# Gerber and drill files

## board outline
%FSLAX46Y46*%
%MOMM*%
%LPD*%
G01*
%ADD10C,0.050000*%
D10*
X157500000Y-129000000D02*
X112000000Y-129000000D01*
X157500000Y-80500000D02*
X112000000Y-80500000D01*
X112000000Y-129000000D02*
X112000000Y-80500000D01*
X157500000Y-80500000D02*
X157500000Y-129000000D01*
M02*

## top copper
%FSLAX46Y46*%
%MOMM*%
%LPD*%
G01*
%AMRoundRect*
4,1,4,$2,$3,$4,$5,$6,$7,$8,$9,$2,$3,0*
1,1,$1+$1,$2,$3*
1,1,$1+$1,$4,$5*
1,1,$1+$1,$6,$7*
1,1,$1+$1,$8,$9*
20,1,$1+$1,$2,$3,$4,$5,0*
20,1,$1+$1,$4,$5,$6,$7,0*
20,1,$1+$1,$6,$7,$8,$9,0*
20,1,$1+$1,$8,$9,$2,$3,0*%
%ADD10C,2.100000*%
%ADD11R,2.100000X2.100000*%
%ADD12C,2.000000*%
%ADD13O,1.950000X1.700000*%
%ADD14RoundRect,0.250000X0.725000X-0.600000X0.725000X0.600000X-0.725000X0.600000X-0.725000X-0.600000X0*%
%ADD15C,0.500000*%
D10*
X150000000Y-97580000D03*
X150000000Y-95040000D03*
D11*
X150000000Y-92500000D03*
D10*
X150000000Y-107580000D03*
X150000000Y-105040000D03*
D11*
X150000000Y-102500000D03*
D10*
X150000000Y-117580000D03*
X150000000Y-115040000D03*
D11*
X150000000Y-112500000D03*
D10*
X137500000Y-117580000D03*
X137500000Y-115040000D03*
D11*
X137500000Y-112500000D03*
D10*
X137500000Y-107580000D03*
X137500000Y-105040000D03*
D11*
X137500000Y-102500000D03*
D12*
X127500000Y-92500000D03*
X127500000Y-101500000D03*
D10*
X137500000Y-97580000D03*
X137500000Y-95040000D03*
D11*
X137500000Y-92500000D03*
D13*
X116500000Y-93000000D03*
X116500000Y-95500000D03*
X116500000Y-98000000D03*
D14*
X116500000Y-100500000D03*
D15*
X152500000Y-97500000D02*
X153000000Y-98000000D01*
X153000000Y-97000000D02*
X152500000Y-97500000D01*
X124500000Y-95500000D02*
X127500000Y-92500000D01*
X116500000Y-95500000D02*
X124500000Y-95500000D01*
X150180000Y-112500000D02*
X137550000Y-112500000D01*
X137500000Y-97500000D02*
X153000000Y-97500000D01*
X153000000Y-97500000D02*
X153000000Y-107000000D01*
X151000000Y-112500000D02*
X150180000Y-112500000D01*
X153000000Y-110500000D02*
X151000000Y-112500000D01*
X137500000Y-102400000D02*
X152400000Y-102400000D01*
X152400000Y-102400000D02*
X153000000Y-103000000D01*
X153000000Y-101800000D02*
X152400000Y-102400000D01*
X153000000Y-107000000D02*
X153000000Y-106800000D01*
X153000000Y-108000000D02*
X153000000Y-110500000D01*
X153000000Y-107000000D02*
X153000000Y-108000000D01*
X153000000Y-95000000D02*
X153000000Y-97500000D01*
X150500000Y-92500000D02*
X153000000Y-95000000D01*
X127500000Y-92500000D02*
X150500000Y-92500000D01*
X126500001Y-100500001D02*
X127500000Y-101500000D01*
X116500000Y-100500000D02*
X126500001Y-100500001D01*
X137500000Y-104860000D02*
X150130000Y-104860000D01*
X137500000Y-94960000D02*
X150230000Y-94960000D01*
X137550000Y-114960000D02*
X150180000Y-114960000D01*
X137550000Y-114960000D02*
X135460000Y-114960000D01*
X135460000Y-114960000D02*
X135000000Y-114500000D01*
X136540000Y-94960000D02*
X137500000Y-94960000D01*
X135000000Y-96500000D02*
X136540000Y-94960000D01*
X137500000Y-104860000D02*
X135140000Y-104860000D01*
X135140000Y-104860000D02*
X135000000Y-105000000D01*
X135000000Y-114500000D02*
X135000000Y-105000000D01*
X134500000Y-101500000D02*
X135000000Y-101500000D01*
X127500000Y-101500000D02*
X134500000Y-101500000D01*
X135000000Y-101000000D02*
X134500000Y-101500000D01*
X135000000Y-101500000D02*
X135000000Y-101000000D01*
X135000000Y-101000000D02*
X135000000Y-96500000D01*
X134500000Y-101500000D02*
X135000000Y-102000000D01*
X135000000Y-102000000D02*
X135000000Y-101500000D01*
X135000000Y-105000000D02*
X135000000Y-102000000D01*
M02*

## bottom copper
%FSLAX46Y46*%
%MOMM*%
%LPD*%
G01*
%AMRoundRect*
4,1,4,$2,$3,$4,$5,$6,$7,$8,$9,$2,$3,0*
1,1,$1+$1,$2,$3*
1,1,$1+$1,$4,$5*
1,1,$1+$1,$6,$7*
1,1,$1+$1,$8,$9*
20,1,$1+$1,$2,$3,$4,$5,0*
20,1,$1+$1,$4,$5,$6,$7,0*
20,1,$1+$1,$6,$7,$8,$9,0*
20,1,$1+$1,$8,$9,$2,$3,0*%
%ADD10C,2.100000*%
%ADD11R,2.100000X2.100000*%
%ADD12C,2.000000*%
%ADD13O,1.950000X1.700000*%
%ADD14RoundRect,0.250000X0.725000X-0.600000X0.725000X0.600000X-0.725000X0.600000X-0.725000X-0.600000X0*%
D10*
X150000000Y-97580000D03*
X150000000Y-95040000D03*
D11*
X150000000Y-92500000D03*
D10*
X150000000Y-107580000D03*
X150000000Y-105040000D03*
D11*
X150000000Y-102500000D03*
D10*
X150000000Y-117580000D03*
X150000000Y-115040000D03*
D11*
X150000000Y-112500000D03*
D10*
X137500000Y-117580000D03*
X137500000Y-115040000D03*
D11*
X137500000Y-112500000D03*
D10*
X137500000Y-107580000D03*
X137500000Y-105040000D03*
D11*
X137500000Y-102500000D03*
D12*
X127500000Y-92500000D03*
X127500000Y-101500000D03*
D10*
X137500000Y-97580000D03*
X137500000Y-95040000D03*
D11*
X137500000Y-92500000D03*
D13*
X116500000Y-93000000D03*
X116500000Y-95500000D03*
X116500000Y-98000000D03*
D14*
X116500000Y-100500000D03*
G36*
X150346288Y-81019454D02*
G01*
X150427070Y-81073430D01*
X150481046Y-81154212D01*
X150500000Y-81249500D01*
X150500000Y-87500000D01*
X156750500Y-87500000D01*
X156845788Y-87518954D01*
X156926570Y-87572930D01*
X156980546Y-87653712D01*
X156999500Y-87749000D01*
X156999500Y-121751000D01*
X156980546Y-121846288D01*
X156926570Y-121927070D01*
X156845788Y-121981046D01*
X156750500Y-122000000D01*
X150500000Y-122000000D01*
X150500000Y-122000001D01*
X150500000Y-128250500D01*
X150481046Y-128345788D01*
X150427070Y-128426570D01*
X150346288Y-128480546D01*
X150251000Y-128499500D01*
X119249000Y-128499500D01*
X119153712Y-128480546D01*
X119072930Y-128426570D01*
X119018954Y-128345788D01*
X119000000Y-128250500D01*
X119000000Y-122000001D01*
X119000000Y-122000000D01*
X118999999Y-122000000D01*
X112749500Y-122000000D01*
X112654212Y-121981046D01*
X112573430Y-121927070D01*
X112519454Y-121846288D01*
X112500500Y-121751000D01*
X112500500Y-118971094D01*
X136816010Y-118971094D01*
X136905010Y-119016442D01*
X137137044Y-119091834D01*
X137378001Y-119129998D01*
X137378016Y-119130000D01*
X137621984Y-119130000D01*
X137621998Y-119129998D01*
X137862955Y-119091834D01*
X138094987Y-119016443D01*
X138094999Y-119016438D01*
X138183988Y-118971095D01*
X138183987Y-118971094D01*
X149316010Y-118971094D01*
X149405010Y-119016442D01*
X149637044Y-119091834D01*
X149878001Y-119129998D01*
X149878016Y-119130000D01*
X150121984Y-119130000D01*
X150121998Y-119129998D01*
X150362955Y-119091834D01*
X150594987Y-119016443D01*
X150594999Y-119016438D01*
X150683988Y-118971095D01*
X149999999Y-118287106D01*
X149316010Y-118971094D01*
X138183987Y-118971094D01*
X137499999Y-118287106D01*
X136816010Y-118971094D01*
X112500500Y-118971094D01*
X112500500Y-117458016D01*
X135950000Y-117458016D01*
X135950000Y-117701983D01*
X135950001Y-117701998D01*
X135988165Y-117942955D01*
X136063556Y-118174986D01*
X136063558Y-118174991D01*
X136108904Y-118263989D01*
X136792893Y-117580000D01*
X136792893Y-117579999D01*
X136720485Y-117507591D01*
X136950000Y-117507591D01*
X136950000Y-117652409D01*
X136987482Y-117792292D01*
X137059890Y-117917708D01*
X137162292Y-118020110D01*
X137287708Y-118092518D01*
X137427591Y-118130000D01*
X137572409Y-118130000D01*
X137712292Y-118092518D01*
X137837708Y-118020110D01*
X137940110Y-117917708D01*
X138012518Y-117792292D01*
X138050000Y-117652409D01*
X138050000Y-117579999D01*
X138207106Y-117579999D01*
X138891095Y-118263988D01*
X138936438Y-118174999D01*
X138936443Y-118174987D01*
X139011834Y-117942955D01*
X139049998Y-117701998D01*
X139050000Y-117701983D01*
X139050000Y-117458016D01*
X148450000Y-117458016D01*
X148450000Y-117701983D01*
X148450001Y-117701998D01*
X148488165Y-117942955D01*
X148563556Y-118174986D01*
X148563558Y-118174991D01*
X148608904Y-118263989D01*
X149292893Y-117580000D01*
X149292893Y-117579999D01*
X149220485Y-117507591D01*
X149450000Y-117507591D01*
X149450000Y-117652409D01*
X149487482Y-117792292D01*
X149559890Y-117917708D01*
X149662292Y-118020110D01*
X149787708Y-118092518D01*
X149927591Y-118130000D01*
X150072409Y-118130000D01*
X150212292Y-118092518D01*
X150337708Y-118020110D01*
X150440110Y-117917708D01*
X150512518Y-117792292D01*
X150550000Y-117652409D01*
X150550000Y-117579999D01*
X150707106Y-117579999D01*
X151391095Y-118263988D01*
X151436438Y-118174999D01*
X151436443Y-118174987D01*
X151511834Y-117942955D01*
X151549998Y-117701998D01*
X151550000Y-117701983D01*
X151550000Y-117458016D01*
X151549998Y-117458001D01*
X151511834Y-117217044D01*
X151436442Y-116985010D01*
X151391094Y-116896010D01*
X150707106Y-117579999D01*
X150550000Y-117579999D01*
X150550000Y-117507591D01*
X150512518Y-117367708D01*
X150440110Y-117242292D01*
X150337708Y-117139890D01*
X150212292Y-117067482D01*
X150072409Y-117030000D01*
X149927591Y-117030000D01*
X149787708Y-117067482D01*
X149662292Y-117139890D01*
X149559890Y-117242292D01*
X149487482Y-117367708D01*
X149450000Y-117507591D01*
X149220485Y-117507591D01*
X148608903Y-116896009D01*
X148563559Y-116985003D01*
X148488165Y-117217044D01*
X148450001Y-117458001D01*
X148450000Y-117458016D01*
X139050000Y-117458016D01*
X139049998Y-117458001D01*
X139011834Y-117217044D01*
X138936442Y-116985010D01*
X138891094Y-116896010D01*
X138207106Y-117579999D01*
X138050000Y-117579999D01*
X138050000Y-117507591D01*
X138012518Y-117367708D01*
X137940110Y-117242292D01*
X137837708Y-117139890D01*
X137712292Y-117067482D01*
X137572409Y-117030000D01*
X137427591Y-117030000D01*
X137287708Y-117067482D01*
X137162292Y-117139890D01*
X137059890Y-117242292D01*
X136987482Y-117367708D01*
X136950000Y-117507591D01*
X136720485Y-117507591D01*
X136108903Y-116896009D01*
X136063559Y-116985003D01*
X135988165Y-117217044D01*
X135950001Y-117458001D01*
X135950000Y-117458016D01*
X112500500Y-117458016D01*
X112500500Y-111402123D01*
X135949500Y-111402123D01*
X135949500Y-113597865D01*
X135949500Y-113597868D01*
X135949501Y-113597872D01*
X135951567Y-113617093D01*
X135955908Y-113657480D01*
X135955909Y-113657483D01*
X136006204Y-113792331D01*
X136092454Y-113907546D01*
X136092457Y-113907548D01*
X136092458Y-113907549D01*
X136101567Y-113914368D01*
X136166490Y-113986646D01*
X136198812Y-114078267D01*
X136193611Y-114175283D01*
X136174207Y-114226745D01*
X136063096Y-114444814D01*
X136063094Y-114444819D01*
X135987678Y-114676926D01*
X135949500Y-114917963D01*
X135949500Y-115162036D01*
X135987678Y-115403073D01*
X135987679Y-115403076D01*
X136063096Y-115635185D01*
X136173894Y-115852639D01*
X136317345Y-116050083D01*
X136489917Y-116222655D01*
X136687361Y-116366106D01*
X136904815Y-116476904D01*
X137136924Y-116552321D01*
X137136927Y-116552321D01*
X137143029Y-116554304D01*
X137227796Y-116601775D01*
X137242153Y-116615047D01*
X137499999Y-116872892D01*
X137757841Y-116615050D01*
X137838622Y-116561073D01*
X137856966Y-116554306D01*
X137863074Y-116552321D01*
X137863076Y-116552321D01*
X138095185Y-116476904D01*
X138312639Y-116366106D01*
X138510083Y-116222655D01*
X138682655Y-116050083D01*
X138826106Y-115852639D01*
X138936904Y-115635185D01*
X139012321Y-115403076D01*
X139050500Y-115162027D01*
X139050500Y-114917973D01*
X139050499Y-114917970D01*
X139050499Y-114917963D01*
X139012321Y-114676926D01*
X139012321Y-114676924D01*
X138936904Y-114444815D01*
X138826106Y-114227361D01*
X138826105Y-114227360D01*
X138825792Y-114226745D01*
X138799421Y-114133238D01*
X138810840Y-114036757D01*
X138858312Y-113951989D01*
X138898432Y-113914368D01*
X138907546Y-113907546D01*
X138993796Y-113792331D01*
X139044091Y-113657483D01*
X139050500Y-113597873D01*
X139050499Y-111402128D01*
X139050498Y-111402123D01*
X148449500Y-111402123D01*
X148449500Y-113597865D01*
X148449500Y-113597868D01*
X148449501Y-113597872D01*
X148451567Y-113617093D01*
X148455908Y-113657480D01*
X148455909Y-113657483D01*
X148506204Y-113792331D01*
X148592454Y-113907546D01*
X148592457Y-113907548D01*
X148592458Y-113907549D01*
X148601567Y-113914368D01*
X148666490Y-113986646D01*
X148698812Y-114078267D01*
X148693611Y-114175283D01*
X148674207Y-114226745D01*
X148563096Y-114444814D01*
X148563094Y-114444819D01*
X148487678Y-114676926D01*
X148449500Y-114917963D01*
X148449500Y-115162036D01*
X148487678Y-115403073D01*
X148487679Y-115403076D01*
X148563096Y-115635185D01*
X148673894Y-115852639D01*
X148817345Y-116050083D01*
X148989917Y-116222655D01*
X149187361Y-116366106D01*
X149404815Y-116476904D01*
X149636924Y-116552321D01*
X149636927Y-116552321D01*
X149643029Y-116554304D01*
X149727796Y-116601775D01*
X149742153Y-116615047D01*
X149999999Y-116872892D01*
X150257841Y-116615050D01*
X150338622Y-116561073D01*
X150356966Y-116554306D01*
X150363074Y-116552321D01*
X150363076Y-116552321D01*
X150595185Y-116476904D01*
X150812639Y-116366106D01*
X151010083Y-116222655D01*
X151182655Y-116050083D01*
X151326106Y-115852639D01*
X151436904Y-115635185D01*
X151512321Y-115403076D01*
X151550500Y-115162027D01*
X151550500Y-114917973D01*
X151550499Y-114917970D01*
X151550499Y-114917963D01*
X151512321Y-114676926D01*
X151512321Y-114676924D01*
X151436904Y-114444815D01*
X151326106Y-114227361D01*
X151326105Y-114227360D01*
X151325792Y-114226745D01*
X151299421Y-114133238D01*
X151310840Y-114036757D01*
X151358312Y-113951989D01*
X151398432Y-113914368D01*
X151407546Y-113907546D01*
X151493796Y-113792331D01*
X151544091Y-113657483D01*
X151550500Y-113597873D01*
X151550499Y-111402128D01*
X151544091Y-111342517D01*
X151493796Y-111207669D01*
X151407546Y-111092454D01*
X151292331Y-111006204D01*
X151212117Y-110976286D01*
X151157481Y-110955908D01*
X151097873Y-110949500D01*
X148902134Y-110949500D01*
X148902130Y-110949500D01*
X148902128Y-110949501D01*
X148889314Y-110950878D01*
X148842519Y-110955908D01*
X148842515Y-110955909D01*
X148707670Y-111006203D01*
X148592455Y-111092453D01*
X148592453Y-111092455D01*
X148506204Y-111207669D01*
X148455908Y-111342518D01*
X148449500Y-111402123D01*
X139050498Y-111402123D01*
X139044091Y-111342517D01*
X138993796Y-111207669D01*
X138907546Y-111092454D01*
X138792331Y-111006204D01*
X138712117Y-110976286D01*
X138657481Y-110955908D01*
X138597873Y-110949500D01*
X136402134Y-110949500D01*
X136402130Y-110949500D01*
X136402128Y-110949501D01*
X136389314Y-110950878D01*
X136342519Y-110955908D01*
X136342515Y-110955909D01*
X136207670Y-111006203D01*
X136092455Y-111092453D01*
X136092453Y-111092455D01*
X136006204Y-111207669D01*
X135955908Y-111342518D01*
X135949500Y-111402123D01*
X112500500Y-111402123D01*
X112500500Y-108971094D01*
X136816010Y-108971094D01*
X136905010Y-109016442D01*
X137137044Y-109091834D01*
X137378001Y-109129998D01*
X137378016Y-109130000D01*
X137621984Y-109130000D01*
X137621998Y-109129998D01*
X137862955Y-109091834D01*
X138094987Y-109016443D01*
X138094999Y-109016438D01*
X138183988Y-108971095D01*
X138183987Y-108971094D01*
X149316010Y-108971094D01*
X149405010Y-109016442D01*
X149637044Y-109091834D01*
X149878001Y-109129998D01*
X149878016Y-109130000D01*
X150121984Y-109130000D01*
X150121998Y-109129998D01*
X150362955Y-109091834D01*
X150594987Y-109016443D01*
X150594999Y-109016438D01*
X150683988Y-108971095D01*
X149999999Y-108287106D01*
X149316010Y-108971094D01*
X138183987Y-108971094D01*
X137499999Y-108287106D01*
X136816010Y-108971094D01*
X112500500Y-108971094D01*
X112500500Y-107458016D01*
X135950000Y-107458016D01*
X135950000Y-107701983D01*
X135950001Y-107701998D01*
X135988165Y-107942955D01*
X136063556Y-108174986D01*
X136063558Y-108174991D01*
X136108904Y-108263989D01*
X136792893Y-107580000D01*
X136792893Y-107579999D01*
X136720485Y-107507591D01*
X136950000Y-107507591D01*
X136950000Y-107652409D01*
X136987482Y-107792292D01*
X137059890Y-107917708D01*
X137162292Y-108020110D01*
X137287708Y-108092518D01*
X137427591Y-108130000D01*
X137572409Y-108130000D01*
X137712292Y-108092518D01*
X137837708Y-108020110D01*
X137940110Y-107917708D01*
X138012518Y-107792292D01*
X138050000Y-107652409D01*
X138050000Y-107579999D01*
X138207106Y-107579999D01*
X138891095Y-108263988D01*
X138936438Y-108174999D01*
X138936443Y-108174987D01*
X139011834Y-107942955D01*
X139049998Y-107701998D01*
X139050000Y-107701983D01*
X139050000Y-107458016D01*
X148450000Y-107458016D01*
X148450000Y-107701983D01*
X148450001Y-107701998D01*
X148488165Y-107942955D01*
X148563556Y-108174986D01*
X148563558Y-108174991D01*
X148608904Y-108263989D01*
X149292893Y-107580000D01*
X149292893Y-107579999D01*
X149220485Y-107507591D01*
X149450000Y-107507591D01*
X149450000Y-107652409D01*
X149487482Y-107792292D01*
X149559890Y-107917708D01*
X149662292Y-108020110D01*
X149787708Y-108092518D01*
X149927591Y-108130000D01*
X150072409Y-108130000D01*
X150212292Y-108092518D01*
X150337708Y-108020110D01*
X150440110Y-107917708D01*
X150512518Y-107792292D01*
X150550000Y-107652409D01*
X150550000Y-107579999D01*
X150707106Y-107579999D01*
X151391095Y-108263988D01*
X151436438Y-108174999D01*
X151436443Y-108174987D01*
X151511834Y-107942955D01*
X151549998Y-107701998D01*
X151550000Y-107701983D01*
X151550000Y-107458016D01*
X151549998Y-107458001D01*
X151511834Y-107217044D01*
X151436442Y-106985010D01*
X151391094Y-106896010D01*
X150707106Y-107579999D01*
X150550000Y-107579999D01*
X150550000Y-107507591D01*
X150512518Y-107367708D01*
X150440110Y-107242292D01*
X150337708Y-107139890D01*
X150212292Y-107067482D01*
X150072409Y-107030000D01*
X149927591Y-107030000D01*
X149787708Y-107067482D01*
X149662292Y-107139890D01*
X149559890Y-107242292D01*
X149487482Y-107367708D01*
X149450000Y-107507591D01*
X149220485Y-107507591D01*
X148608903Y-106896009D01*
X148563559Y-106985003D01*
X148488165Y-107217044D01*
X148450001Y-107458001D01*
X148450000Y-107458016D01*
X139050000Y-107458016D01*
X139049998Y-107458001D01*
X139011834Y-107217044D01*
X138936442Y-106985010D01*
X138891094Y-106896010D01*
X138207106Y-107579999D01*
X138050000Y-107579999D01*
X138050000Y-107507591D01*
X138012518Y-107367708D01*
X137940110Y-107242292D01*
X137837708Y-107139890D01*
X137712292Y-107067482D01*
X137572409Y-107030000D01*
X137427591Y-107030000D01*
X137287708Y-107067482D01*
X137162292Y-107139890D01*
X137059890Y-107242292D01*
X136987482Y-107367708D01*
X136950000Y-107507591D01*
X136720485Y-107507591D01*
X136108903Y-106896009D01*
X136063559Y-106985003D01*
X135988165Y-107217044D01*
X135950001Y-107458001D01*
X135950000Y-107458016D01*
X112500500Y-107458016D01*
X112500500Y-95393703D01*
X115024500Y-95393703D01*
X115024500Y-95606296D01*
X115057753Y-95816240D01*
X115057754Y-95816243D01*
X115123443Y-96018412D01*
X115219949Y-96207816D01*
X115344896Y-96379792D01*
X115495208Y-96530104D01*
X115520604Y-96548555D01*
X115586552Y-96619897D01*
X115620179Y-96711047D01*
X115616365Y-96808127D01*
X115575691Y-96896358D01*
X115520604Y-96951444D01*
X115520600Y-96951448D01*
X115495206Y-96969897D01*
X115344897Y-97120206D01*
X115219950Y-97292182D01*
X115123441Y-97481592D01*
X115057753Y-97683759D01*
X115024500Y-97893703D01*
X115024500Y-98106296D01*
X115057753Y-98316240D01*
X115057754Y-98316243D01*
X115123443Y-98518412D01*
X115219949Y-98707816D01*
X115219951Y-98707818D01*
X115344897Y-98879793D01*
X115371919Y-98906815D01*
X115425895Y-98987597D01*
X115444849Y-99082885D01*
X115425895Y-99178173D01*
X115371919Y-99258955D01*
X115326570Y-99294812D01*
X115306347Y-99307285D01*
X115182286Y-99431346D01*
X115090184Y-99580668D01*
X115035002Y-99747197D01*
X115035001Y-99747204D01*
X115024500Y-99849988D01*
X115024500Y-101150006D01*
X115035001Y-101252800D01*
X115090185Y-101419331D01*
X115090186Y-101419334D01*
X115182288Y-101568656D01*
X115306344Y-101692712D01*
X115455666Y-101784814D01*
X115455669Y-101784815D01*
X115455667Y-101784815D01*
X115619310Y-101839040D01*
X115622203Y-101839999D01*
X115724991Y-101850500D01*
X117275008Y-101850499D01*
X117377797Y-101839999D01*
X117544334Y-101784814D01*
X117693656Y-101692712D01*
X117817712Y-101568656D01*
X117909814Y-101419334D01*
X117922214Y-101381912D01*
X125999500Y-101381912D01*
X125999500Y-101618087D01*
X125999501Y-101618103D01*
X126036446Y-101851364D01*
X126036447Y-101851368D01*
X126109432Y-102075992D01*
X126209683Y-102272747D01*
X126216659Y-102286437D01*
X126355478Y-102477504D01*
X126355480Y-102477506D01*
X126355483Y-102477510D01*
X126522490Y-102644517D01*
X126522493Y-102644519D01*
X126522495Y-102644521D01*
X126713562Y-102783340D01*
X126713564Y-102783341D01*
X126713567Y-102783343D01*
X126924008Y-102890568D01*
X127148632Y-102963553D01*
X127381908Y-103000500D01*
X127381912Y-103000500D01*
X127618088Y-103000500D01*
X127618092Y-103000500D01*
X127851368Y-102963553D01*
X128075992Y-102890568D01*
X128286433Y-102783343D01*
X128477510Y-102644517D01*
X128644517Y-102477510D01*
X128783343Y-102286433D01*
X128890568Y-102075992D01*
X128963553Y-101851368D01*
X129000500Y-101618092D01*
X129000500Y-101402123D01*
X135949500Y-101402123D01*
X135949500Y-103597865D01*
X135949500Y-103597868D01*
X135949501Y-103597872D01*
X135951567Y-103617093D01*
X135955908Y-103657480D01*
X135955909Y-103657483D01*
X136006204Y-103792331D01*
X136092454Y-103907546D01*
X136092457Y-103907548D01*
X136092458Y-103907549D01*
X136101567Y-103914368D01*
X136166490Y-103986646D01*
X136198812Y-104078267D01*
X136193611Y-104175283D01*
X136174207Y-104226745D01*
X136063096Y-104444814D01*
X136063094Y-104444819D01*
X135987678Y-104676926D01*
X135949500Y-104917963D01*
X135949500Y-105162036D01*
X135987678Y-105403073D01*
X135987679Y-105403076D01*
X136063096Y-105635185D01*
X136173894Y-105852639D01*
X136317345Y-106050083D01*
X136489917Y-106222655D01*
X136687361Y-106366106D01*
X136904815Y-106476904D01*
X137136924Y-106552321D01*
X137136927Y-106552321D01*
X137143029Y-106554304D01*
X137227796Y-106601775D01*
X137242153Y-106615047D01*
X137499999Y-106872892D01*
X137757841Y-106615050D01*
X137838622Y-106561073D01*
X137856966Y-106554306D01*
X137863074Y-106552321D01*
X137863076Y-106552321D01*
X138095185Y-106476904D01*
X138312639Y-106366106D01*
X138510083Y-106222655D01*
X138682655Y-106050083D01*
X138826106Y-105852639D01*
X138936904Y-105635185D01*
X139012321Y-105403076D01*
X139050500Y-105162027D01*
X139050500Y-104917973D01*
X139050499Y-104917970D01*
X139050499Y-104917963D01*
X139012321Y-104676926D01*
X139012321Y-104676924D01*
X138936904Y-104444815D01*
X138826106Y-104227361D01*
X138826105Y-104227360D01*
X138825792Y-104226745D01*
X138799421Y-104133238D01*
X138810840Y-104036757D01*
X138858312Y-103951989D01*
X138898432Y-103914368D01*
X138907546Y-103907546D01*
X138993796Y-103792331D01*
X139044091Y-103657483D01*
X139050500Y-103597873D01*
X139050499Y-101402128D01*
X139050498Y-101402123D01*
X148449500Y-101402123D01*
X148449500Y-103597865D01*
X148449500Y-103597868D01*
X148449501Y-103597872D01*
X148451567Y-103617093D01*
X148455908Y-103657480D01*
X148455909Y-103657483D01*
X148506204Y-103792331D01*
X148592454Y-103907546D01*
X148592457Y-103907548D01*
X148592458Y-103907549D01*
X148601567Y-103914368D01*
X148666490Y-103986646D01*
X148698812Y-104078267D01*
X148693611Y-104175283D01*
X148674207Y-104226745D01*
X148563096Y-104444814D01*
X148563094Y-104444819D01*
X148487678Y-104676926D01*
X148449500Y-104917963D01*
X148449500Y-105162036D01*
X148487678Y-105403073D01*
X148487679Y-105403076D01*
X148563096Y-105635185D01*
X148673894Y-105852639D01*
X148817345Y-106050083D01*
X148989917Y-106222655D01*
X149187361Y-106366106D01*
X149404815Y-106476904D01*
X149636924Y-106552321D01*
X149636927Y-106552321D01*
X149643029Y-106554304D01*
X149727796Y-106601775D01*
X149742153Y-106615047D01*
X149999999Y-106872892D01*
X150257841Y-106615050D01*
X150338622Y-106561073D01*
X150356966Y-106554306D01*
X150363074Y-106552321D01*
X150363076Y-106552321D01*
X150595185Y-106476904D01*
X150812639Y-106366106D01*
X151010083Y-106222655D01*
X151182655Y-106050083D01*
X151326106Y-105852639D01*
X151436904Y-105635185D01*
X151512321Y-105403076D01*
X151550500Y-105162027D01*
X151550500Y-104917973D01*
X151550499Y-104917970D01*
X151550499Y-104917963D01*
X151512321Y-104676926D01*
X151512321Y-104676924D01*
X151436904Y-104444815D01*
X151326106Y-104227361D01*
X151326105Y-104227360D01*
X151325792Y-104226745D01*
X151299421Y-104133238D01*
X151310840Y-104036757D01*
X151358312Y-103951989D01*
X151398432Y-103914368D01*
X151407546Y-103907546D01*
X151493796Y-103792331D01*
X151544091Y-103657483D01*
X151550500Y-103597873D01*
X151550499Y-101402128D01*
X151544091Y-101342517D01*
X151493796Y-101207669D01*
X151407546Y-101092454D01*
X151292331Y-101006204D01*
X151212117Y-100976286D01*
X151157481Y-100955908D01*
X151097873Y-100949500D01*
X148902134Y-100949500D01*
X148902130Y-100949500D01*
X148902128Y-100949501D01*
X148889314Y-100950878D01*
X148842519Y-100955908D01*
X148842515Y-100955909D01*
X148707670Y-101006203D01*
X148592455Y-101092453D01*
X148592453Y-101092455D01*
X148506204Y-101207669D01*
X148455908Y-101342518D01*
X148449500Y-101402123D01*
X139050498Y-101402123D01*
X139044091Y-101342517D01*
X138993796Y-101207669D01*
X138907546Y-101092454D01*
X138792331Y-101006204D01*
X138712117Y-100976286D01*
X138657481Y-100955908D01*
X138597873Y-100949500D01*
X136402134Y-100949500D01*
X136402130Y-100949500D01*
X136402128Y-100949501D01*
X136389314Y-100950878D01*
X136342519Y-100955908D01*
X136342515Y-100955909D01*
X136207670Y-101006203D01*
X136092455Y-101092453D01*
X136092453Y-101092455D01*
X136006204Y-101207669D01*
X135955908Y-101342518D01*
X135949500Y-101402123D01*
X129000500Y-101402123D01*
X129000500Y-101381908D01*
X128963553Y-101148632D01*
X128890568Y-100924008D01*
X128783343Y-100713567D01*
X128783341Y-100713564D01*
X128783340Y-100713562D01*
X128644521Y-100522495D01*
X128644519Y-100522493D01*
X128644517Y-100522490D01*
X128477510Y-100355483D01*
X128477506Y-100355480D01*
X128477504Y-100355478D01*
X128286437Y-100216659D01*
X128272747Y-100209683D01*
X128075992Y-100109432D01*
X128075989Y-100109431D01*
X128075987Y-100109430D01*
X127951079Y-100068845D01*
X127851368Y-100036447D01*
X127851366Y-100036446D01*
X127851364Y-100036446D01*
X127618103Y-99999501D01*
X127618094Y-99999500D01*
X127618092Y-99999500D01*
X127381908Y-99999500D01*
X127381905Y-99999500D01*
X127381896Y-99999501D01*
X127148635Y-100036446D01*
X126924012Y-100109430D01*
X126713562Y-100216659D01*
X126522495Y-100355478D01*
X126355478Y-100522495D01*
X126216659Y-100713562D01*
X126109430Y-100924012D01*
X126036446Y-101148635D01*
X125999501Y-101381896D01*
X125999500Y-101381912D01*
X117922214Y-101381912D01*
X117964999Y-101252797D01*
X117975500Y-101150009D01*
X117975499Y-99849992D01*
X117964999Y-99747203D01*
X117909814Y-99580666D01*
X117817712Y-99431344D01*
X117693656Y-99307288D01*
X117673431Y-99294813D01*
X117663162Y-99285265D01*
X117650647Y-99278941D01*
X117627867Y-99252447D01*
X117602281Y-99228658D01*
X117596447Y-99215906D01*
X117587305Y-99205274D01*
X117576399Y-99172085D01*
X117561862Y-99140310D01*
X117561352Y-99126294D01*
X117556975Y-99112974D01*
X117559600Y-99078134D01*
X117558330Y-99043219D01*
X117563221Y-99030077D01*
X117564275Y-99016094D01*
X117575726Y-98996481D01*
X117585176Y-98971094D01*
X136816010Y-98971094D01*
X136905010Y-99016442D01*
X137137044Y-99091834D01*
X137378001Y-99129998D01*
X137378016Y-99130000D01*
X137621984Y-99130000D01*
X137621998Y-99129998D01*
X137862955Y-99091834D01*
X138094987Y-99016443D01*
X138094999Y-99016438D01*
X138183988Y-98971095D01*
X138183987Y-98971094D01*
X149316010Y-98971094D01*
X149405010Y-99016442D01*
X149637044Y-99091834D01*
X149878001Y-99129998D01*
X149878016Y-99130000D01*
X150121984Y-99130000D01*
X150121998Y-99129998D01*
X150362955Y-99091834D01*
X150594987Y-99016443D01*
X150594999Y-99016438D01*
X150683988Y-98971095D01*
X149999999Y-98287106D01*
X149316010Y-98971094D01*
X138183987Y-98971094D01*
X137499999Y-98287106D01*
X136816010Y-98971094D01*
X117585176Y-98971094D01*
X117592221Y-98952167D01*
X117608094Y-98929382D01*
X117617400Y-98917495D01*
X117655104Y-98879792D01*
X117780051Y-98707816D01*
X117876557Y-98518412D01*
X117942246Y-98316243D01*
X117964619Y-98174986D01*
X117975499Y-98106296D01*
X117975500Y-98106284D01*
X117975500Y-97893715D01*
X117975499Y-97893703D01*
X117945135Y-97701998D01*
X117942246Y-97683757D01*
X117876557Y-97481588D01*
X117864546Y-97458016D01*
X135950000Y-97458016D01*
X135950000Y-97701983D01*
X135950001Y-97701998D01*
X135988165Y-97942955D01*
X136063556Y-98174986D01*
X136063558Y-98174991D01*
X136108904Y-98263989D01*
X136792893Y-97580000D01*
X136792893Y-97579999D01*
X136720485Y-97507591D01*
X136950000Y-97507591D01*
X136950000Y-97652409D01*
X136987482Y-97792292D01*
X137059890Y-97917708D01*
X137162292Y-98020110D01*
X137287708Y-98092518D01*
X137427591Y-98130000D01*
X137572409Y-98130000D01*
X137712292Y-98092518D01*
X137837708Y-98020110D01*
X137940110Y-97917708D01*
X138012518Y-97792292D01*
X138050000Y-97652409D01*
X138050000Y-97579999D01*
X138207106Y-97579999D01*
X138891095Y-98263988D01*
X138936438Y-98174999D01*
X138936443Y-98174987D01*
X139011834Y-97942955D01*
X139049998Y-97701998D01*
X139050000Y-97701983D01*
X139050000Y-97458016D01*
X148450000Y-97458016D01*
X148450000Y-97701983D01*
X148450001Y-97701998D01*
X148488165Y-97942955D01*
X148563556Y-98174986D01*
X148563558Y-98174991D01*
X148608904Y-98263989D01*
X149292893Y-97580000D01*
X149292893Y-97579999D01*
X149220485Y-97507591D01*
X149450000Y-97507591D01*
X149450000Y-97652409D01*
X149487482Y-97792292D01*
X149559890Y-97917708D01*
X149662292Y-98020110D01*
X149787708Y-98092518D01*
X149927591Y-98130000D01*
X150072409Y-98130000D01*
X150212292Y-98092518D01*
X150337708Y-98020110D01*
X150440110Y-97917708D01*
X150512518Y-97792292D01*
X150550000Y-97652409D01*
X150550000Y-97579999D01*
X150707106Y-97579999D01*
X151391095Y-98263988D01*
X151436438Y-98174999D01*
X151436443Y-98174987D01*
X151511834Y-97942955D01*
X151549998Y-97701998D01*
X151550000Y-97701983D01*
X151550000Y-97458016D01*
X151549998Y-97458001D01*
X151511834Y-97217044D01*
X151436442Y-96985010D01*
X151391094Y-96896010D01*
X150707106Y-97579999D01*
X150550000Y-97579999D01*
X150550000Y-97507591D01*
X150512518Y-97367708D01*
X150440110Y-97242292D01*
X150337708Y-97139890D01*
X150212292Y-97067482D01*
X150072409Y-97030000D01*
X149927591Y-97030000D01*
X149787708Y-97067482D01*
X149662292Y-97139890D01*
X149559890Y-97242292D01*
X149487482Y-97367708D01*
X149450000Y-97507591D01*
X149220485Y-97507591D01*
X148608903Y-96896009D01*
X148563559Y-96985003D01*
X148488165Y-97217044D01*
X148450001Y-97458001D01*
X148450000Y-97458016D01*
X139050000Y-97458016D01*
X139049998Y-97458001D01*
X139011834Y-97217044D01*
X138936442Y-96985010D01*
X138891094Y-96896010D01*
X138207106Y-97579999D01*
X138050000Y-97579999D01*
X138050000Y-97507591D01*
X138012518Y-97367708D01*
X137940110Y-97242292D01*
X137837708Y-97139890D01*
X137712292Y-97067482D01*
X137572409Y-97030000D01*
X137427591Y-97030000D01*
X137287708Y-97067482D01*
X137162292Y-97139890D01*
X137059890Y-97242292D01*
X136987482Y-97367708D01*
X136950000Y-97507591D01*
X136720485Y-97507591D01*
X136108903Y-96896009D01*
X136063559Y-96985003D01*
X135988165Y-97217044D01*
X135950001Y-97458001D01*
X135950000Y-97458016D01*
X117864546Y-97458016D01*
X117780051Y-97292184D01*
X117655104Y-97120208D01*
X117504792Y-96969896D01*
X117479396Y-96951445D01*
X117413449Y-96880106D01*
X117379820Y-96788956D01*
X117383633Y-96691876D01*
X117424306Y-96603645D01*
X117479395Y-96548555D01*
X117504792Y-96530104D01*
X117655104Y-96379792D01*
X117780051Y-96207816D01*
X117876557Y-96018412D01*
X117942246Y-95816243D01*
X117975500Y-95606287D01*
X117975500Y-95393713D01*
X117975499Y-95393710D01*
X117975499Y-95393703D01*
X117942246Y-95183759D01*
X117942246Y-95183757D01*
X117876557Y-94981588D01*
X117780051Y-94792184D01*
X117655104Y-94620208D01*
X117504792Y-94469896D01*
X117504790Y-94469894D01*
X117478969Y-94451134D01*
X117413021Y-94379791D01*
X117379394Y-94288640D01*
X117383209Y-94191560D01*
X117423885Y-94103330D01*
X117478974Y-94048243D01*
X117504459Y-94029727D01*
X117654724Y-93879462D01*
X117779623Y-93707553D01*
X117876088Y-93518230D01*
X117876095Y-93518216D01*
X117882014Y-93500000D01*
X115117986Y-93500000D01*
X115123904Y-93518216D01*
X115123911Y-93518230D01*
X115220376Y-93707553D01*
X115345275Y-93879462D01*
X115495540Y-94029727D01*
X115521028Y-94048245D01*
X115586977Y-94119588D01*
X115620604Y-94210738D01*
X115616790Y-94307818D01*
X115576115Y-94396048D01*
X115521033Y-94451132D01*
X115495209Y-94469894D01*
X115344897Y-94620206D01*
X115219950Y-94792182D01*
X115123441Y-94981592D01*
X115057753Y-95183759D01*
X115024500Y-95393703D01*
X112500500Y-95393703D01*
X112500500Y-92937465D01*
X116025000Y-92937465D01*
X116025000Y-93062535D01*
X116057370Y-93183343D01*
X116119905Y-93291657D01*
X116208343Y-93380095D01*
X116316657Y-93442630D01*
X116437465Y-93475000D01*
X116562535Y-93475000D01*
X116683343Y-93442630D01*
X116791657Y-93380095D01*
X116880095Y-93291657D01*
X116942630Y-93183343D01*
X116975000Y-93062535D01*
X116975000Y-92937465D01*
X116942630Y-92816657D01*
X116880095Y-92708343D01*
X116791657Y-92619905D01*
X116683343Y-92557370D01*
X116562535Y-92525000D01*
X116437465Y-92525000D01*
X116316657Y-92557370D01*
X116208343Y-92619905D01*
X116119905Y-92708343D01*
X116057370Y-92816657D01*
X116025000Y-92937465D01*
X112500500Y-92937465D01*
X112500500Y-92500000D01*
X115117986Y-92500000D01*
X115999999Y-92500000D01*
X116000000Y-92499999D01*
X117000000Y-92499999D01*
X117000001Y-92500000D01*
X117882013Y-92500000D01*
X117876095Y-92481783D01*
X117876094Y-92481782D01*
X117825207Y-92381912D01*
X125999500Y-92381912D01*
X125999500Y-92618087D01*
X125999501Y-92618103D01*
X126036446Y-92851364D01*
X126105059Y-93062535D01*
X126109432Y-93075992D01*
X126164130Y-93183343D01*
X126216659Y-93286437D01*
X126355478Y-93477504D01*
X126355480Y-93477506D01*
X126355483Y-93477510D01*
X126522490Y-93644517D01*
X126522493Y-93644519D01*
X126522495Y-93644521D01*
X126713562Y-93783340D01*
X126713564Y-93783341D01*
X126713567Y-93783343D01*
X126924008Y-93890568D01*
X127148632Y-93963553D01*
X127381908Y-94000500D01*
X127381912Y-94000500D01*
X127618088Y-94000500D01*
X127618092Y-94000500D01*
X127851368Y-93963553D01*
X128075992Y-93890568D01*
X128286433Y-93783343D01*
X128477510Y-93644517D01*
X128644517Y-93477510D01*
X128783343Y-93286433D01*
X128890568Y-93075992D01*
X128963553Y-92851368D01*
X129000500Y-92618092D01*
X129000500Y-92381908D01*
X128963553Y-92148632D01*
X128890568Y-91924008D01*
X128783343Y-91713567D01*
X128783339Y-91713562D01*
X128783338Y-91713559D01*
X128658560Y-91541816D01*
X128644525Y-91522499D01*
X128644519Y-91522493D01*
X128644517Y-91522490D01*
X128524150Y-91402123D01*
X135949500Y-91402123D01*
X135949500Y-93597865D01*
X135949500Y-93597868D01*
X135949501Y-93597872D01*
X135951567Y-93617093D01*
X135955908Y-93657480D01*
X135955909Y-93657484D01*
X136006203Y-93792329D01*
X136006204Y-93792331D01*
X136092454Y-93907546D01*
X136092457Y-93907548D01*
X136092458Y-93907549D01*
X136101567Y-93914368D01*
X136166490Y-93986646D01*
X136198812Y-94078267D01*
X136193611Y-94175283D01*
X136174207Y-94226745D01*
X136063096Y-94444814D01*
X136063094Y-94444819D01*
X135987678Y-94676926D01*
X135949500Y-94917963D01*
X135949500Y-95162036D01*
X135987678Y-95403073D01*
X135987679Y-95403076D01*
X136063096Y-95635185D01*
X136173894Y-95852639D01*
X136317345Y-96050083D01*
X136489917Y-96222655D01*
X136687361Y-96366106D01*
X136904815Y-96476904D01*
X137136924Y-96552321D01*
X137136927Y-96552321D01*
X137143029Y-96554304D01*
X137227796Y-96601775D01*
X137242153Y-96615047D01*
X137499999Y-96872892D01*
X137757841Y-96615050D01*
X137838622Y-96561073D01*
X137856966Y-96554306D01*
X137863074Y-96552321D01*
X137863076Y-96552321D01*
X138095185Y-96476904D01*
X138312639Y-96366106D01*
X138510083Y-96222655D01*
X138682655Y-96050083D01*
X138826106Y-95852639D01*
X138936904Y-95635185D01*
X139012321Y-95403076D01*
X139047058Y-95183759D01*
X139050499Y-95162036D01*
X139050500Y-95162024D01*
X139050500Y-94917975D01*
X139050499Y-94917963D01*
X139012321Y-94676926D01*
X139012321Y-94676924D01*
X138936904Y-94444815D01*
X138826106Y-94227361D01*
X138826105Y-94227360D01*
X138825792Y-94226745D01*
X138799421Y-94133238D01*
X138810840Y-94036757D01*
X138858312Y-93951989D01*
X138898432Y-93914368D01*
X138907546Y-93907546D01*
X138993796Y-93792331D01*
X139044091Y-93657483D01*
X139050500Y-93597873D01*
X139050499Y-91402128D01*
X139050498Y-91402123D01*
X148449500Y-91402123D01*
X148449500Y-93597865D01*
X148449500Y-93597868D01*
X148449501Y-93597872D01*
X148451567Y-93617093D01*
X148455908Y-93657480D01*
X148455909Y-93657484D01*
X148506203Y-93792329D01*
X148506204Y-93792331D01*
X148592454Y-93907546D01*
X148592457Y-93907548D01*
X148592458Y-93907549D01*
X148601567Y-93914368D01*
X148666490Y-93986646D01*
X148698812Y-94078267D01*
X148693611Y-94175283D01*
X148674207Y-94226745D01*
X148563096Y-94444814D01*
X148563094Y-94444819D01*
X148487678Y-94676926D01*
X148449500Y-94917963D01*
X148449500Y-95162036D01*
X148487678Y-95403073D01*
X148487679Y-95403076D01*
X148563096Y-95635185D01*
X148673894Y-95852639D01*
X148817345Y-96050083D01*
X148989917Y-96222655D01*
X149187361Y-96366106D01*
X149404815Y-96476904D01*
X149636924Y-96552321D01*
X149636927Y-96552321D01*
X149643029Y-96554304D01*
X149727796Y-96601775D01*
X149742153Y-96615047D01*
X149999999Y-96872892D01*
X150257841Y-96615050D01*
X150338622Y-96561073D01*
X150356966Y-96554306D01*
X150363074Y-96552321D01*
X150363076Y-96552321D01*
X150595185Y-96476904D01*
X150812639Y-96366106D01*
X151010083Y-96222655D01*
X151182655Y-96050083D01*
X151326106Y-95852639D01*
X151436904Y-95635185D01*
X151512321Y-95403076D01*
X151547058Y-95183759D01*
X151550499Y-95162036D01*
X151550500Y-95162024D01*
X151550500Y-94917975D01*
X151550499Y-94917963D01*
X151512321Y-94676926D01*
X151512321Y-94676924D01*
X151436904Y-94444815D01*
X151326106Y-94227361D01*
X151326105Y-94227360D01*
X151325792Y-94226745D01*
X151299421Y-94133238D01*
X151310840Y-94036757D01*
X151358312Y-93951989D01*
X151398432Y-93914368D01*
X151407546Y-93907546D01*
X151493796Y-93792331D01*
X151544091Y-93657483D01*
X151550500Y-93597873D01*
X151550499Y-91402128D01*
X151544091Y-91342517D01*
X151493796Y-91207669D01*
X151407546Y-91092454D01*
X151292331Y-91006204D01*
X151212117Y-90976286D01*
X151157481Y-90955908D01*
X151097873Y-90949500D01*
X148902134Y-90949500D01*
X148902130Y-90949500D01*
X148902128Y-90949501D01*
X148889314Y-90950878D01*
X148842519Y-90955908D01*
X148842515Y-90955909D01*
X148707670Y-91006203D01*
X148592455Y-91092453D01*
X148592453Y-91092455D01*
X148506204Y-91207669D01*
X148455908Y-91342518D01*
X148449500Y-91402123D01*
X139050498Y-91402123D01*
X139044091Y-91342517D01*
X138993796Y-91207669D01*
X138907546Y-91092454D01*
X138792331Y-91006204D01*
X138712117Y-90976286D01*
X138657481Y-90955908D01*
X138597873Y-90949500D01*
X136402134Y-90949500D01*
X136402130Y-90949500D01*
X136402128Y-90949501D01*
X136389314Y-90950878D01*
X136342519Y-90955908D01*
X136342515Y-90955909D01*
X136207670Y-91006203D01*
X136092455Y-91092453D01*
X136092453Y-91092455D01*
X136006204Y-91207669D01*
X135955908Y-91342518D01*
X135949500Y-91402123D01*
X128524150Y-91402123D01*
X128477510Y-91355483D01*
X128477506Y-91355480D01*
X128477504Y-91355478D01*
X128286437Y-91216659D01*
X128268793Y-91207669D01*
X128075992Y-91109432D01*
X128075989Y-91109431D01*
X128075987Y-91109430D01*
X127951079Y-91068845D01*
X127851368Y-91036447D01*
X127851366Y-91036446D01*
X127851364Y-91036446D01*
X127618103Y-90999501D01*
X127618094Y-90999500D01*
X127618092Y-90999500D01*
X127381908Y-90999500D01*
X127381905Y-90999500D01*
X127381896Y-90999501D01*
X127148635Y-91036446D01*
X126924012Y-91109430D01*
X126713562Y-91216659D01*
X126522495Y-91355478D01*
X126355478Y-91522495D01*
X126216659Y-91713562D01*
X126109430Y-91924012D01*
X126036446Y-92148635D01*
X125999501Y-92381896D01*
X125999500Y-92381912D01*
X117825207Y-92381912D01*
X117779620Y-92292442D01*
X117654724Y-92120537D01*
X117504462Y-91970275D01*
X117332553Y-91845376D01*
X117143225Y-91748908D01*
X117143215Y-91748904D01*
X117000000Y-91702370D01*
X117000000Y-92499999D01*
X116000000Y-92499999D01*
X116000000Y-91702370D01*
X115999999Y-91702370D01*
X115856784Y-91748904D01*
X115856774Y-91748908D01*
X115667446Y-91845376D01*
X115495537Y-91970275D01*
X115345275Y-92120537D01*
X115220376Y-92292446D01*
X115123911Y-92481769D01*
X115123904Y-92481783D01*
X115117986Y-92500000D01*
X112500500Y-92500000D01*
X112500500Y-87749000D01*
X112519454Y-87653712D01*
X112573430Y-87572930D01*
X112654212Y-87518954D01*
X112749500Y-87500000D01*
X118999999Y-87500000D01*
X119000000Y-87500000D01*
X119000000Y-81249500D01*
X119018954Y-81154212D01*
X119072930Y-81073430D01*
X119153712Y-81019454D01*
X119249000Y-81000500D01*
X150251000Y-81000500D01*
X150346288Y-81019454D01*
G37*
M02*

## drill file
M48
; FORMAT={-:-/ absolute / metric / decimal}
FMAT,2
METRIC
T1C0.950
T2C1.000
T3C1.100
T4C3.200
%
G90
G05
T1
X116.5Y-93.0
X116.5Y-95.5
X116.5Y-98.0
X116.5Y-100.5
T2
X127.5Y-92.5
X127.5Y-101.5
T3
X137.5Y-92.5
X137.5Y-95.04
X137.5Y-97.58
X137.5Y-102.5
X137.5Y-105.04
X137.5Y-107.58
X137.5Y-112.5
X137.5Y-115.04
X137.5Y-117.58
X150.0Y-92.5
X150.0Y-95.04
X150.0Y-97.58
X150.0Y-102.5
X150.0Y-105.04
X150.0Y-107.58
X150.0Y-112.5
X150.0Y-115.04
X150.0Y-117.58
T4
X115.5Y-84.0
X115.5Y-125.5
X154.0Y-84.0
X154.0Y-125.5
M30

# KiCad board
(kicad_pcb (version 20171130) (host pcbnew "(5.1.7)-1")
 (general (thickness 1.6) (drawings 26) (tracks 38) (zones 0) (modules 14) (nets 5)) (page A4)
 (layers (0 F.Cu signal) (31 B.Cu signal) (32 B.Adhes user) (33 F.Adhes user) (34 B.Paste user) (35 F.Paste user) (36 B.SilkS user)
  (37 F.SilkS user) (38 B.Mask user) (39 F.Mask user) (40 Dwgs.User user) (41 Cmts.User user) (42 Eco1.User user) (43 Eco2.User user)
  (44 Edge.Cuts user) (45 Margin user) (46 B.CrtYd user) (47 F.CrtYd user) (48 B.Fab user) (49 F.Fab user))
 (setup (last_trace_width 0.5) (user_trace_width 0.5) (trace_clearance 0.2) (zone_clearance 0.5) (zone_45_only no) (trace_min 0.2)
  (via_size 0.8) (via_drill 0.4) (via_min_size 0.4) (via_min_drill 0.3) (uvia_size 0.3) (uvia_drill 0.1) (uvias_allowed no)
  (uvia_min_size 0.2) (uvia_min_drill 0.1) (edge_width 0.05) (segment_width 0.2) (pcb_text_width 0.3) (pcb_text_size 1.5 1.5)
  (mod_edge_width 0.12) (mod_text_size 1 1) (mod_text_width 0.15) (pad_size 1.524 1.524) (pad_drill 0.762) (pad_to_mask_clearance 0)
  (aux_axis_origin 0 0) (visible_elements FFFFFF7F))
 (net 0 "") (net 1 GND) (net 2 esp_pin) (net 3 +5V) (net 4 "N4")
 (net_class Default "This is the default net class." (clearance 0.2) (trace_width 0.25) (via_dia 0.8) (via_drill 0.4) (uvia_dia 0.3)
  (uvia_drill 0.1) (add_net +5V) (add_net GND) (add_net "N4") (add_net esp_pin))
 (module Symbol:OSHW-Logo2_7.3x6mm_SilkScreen (layer F.Cu) (at 137.5 124.5)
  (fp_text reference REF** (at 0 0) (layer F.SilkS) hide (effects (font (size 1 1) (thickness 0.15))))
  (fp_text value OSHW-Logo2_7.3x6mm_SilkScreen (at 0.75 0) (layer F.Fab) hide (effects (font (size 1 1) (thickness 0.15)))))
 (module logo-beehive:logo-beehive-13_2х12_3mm (layer F.Cu) (at 123 112.5)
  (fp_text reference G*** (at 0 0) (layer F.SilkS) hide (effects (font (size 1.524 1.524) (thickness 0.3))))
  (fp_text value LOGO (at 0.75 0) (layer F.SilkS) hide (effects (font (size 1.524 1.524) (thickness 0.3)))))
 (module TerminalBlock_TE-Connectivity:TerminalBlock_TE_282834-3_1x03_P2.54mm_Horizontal (layer F.Cu) (at 150 92.5 270)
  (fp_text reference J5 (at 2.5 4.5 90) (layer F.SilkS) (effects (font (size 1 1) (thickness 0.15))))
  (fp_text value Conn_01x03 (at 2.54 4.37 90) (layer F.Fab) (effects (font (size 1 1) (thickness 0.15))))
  (pad 3 thru_hole circle (at 5.08 0 270) (size 2.1 2.1) (drill 1.1) (layers *.Cu *.Mask) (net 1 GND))
  (pad 2 thru_hole circle (at 2.54 0 270) (size 2.1 2.1) (drill 1.1) (layers *.Cu *.Mask) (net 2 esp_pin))
  (pad 1 thru_hole rect (at 0 0 270) (size 2.1 2.1) (drill 1.1) (layers *.Cu *.Mask) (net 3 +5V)))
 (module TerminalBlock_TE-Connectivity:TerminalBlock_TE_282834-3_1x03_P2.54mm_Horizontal (layer F.Cu) (at 150 102.5 270)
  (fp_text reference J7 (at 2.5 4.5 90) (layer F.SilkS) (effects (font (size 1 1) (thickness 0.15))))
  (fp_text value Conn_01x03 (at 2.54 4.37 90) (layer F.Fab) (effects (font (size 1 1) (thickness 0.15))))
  (pad 3 thru_hole circle (at 5.08 0 270) (size 2.1 2.1) (drill 1.1) (layers *.Cu *.Mask) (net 1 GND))
  (pad 2 thru_hole circle (at 2.54 0 270) (size 2.1 2.1) (drill 1.1) (layers *.Cu *.Mask) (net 2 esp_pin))
  (pad 1 thru_hole rect (at 0 0 270) (size 2.1 2.1) (drill 1.1) (layers *.Cu *.Mask) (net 3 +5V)))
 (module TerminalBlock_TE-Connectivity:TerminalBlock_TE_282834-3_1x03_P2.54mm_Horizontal (layer F.Cu) (at 150 112.5 270)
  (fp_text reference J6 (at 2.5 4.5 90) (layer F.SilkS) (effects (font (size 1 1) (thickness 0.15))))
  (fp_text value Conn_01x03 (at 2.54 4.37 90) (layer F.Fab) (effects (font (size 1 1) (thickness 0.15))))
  (pad 3 thru_hole circle (at 5.08 0 270) (size 2.1 2.1) (drill 1.1) (layers *.Cu *.Mask) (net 1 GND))
  (pad 2 thru_hole circle (at 2.54 0 270) (size 2.1 2.1) (drill 1.1) (layers *.Cu *.Mask) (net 2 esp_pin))
  (pad 1 thru_hole rect (at 0 0 270) (size 2.1 2.1) (drill 1.1) (layers *.Cu *.Mask) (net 3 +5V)))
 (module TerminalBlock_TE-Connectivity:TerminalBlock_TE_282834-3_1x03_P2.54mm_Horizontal (layer F.Cu) (at 137.5 112.5 270)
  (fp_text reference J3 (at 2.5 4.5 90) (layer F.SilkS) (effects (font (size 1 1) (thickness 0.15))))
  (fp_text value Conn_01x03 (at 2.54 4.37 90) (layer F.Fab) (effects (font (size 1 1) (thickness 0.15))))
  (pad 3 thru_hole circle (at 5.08 0 270) (size 2.1 2.1) (drill 1.1) (layers *.Cu *.Mask) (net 1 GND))
  (pad 2 thru_hole circle (at 2.54 0 270) (size 2.1 2.1) (drill 1.1) (layers *.Cu *.Mask) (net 2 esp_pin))
  (pad 1 thru_hole rect (at 0 0 270) (size 2.1 2.1) (drill 1.1) (layers *.Cu *.Mask) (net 3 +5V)))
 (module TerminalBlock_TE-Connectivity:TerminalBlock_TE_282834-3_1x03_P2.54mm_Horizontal (layer F.Cu) (at 137.5 102.5 270)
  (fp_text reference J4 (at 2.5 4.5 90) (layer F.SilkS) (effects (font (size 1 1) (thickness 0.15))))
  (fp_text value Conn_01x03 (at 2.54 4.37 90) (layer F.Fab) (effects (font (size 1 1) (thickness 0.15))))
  (pad 3 thru_hole circle (at 5.08 0 270) (size 2.1 2.1) (drill 1.1) (layers *.Cu *.Mask) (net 1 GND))
  (pad 2 thru_hole circle (at 2.54 0 270) (size 2.1 2.1) (drill 1.1) (layers *.Cu *.Mask) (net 2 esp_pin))
  (pad 1 thru_hole rect (at 0 0 270) (size 2.1 2.1) (drill 1.1) (layers *.Cu *.Mask) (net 3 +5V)))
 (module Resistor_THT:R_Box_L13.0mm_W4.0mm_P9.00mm (layer F.Cu) (at 127.5 101.5 90)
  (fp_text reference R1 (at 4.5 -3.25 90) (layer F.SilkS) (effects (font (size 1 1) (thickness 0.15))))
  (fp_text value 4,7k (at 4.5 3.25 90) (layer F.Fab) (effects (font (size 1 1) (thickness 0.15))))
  (pad 2 thru_hole circle (at 9 0 90) (size 2 2) (drill 1) (layers *.Cu *.Mask) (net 3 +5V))
  (pad 1 thru_hole circle (at 0 0 90) (size 2 2) (drill 1) (layers *.Cu *.Mask) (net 2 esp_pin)))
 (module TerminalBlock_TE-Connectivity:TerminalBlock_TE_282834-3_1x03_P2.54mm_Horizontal (layer F.Cu) (at 137.5 92.5 270)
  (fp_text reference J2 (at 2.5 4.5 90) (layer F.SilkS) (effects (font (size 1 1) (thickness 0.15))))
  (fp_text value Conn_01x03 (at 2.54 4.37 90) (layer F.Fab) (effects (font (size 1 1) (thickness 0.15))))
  (pad 3 thru_hole circle (at 5.08 0 270) (size 2.1 2.1) (drill 1.1) (layers *.Cu *.Mask) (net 1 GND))
  (pad 2 thru_hole circle (at 2.54 0 270) (size 2.1 2.1) (drill 1.1) (layers *.Cu *.Mask) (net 2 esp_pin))
  (pad 1 thru_hole rect (at 0 0 270) (size 2.1 2.1) (drill 1.1) (layers *.Cu *.Mask) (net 3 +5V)))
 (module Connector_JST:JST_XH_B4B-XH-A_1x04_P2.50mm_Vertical (layer F.Cu) (at 116.5 100.5 90)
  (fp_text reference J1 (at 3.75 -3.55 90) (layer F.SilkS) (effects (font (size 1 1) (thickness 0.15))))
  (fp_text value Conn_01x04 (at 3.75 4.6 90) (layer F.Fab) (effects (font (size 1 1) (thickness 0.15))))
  (pad 4 thru_hole oval (at 7.5 0 90) (size 1.7 1.95) (drill 0.95) (layers *.Cu *.Mask) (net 1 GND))
  (pad 3 thru_hole oval (at 5 0 90) (size 1.7 1.95) (drill 0.95) (layers *.Cu *.Mask) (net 3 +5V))
  (pad 2 thru_hole oval (at 2.5 0 90) (size 1.7 1.95) (drill 0.95) (layers *.Cu *.Mask) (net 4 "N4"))
  (pad 1 thru_hole roundrect (at 0 0 90) (size 1.7 1.95) (drill 0.95) (layers *.Cu *.Mask) (roundrect_rratio 0.1470588235294118)
   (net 2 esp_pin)))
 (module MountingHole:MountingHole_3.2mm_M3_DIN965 (layer F.Cu) (at 154 125.5)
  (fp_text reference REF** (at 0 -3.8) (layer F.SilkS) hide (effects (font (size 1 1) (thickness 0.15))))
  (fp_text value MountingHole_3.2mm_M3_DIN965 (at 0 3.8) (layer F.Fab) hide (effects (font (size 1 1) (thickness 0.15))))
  (pad 1 np_thru_hole circle (at 0 0) (size 3.2 3.2) (drill 3.2) (layers *.Cu *.Mask)))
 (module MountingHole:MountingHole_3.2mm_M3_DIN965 (layer F.Cu) (at 154 84)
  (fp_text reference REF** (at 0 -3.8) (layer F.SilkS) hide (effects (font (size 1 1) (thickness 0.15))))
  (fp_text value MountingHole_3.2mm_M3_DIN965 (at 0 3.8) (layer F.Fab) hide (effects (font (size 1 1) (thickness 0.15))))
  (pad 1 np_thru_hole circle (at 0 0) (size 3.2 3.2) (drill 3.2) (layers *.Cu *.Mask)))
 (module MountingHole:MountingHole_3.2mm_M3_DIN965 (layer F.Cu) (at 115.5 125.5)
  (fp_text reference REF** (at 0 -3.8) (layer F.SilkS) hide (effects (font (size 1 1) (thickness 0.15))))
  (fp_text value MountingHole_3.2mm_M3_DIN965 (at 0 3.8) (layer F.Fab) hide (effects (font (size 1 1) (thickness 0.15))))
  (pad 1 np_thru_hole circle (at 0 0) (size 3.2 3.2) (drill 3.2) (layers *.Cu *.Mask)))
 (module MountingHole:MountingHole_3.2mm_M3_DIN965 (layer F.Cu) (at 115.5 84)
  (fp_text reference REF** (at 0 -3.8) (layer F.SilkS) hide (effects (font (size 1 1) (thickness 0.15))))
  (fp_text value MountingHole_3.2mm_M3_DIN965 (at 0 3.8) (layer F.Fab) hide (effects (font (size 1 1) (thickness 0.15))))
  (pad 1 np_thru_hole circle (at 0 0) (size 3.2 3.2) (drill 3.2) (layers *.Cu *.Mask)))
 (gr_line (start 157.5 129) (end 112 129) (layer Edge.Cuts) (width 0.05))
 (gr_line (start 157.5 80.5) (end 112 80.5) (layer Edge.Cuts) (width 0.05))
 (gr_line (start 112 129) (end 112 80.5) (layer Edge.Cuts) (width 0.05))
 (gr_line (start 157.5 80.5) (end 157.5 129) (layer Edge.Cuts) (width 0.05))
 (segment (start 152.5 97.5) (end 153 98) (width 0.5) (layer F.Cu) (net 3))
 (segment (start 153 97) (end 152.5 97.5) (width 0.5) (layer F.Cu) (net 3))
 (segment (start 124.5 95.5) (end 127.5 92.5) (width 0.5) (layer F.Cu) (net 3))
 (segment (start 116.5 95.5) (end 124.5 95.5) (width 0.5) (layer F.Cu) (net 3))
 (segment (start 150.18 112.5) (end 137.55 112.5) (width 0.5) (layer F.Cu) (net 3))
 (segment (start 137.5 97.5) (end 153 97.5) (width 0.5) (layer F.Cu) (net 3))
 (segment (start 153 97.5) (end 153 107) (width 0.5) (layer F.Cu) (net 3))
 (segment (start 151 112.5) (end 150.18 112.5) (width 0.5) (layer F.Cu) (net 3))
 (segment (start 153 110.5) (end 151 112.5) (width 0.5) (layer F.Cu) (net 3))
 (segment (start 137.5 102.4) (end 152.4 102.4) (width 0.5) (layer F.Cu) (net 3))
 (segment (start 152.4 102.4) (end 153 103) (width 0.5) (layer F.Cu) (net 3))
 (segment (start 153 101.8) (end 152.4 102.4) (width 0.5) (layer F.Cu) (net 3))
 (segment (start 153 107) (end 153 106.8) (width 0.5) (layer F.Cu) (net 3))
 (segment (start 153 108) (end 153 110.5) (width 0.5) (layer F.Cu) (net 3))
 (segment (start 153 107) (end 153 108) (width 0.5) (layer F.Cu) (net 3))
 (segment (start 153 95) (end 153 97.5) (width 0.5) (layer F.Cu) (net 3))
 (segment (start 150.5 92.5) (end 153 95) (width 0.5) (layer F.Cu) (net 3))
 (segment (start 127.5 92.5) (end 150.5 92.5) (width 0.5) (layer F.Cu) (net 3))
 (segment (start 126.500001 100.500001) (end 127.5 101.5) (width 0.5) (layer F.Cu) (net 2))
 (segment (start 116.5 100.5) (end 126.500001 100.500001) (width 0.5) (layer F.Cu) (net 2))
 (segment (start 137.5 104.86) (end 150.13 104.86) (width 0.5) (layer F.Cu) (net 2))
 (segment (start 137.5 94.96) (end 150.23 94.96) (width 0.5) (layer F.Cu) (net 2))
 (segment (start 137.55 114.96) (end 150.18 114.96) (width 0.5) (layer F.Cu) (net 2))
 (segment (start 137.55 114.96) (end 135.46 114.96) (width 0.5) (layer F.Cu) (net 2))
 (segment (start 135.46 114.96) (end 135 114.5) (width 0.5) (layer F.Cu) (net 2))
 (segment (start 136.54 94.96) (end 137.5 94.96) (width 0.5) (layer F.Cu) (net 2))
 (segment (start 135 96.5) (end 136.54 94.96) (width 0.5) (layer F.Cu) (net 2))
 (segment (start 137.5 104.86) (end 135.14 104.86) (width 0.5) (layer F.Cu) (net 2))
 (segment (start 135.14 104.86) (end 135 105) (width 0.5) (layer F.Cu) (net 2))
 (segment (start 135 114.5) (end 135 105) (width 0.5) (layer F.Cu) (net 2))
 (segment (start 134.5 101.5) (end 135 101.5) (width 0.5) (layer F.Cu) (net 2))
 (segment (start 127.5 101.5) (end 134.5 101.5) (width 0.5) (layer F.Cu) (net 2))
 (segment (start 135 101) (end 134.5 101.5) (width 0.5) (layer F.Cu) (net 2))
 (segment (start 135 101.5) (end 135 101) (width 0.5) (layer F.Cu) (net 2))
 (segment (start 135 101) (end 135 96.5) (width 0.5) (layer F.Cu) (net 2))
 (segment (start 134.5 101.5) (end 135 102) (width 0.5) (layer F.Cu) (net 2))
 (segment (start 135 102) (end 135 101.5) (width 0.5) (layer F.Cu) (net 2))
 (segment (start 135 105) (end 135 102) (width 0.5) (layer F.Cu) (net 2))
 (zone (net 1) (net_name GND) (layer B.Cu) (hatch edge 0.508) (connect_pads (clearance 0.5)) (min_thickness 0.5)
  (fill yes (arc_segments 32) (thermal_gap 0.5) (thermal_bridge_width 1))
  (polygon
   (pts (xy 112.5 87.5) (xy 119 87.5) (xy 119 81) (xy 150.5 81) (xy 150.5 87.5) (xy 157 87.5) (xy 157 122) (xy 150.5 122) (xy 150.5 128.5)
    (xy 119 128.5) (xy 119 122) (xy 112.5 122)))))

